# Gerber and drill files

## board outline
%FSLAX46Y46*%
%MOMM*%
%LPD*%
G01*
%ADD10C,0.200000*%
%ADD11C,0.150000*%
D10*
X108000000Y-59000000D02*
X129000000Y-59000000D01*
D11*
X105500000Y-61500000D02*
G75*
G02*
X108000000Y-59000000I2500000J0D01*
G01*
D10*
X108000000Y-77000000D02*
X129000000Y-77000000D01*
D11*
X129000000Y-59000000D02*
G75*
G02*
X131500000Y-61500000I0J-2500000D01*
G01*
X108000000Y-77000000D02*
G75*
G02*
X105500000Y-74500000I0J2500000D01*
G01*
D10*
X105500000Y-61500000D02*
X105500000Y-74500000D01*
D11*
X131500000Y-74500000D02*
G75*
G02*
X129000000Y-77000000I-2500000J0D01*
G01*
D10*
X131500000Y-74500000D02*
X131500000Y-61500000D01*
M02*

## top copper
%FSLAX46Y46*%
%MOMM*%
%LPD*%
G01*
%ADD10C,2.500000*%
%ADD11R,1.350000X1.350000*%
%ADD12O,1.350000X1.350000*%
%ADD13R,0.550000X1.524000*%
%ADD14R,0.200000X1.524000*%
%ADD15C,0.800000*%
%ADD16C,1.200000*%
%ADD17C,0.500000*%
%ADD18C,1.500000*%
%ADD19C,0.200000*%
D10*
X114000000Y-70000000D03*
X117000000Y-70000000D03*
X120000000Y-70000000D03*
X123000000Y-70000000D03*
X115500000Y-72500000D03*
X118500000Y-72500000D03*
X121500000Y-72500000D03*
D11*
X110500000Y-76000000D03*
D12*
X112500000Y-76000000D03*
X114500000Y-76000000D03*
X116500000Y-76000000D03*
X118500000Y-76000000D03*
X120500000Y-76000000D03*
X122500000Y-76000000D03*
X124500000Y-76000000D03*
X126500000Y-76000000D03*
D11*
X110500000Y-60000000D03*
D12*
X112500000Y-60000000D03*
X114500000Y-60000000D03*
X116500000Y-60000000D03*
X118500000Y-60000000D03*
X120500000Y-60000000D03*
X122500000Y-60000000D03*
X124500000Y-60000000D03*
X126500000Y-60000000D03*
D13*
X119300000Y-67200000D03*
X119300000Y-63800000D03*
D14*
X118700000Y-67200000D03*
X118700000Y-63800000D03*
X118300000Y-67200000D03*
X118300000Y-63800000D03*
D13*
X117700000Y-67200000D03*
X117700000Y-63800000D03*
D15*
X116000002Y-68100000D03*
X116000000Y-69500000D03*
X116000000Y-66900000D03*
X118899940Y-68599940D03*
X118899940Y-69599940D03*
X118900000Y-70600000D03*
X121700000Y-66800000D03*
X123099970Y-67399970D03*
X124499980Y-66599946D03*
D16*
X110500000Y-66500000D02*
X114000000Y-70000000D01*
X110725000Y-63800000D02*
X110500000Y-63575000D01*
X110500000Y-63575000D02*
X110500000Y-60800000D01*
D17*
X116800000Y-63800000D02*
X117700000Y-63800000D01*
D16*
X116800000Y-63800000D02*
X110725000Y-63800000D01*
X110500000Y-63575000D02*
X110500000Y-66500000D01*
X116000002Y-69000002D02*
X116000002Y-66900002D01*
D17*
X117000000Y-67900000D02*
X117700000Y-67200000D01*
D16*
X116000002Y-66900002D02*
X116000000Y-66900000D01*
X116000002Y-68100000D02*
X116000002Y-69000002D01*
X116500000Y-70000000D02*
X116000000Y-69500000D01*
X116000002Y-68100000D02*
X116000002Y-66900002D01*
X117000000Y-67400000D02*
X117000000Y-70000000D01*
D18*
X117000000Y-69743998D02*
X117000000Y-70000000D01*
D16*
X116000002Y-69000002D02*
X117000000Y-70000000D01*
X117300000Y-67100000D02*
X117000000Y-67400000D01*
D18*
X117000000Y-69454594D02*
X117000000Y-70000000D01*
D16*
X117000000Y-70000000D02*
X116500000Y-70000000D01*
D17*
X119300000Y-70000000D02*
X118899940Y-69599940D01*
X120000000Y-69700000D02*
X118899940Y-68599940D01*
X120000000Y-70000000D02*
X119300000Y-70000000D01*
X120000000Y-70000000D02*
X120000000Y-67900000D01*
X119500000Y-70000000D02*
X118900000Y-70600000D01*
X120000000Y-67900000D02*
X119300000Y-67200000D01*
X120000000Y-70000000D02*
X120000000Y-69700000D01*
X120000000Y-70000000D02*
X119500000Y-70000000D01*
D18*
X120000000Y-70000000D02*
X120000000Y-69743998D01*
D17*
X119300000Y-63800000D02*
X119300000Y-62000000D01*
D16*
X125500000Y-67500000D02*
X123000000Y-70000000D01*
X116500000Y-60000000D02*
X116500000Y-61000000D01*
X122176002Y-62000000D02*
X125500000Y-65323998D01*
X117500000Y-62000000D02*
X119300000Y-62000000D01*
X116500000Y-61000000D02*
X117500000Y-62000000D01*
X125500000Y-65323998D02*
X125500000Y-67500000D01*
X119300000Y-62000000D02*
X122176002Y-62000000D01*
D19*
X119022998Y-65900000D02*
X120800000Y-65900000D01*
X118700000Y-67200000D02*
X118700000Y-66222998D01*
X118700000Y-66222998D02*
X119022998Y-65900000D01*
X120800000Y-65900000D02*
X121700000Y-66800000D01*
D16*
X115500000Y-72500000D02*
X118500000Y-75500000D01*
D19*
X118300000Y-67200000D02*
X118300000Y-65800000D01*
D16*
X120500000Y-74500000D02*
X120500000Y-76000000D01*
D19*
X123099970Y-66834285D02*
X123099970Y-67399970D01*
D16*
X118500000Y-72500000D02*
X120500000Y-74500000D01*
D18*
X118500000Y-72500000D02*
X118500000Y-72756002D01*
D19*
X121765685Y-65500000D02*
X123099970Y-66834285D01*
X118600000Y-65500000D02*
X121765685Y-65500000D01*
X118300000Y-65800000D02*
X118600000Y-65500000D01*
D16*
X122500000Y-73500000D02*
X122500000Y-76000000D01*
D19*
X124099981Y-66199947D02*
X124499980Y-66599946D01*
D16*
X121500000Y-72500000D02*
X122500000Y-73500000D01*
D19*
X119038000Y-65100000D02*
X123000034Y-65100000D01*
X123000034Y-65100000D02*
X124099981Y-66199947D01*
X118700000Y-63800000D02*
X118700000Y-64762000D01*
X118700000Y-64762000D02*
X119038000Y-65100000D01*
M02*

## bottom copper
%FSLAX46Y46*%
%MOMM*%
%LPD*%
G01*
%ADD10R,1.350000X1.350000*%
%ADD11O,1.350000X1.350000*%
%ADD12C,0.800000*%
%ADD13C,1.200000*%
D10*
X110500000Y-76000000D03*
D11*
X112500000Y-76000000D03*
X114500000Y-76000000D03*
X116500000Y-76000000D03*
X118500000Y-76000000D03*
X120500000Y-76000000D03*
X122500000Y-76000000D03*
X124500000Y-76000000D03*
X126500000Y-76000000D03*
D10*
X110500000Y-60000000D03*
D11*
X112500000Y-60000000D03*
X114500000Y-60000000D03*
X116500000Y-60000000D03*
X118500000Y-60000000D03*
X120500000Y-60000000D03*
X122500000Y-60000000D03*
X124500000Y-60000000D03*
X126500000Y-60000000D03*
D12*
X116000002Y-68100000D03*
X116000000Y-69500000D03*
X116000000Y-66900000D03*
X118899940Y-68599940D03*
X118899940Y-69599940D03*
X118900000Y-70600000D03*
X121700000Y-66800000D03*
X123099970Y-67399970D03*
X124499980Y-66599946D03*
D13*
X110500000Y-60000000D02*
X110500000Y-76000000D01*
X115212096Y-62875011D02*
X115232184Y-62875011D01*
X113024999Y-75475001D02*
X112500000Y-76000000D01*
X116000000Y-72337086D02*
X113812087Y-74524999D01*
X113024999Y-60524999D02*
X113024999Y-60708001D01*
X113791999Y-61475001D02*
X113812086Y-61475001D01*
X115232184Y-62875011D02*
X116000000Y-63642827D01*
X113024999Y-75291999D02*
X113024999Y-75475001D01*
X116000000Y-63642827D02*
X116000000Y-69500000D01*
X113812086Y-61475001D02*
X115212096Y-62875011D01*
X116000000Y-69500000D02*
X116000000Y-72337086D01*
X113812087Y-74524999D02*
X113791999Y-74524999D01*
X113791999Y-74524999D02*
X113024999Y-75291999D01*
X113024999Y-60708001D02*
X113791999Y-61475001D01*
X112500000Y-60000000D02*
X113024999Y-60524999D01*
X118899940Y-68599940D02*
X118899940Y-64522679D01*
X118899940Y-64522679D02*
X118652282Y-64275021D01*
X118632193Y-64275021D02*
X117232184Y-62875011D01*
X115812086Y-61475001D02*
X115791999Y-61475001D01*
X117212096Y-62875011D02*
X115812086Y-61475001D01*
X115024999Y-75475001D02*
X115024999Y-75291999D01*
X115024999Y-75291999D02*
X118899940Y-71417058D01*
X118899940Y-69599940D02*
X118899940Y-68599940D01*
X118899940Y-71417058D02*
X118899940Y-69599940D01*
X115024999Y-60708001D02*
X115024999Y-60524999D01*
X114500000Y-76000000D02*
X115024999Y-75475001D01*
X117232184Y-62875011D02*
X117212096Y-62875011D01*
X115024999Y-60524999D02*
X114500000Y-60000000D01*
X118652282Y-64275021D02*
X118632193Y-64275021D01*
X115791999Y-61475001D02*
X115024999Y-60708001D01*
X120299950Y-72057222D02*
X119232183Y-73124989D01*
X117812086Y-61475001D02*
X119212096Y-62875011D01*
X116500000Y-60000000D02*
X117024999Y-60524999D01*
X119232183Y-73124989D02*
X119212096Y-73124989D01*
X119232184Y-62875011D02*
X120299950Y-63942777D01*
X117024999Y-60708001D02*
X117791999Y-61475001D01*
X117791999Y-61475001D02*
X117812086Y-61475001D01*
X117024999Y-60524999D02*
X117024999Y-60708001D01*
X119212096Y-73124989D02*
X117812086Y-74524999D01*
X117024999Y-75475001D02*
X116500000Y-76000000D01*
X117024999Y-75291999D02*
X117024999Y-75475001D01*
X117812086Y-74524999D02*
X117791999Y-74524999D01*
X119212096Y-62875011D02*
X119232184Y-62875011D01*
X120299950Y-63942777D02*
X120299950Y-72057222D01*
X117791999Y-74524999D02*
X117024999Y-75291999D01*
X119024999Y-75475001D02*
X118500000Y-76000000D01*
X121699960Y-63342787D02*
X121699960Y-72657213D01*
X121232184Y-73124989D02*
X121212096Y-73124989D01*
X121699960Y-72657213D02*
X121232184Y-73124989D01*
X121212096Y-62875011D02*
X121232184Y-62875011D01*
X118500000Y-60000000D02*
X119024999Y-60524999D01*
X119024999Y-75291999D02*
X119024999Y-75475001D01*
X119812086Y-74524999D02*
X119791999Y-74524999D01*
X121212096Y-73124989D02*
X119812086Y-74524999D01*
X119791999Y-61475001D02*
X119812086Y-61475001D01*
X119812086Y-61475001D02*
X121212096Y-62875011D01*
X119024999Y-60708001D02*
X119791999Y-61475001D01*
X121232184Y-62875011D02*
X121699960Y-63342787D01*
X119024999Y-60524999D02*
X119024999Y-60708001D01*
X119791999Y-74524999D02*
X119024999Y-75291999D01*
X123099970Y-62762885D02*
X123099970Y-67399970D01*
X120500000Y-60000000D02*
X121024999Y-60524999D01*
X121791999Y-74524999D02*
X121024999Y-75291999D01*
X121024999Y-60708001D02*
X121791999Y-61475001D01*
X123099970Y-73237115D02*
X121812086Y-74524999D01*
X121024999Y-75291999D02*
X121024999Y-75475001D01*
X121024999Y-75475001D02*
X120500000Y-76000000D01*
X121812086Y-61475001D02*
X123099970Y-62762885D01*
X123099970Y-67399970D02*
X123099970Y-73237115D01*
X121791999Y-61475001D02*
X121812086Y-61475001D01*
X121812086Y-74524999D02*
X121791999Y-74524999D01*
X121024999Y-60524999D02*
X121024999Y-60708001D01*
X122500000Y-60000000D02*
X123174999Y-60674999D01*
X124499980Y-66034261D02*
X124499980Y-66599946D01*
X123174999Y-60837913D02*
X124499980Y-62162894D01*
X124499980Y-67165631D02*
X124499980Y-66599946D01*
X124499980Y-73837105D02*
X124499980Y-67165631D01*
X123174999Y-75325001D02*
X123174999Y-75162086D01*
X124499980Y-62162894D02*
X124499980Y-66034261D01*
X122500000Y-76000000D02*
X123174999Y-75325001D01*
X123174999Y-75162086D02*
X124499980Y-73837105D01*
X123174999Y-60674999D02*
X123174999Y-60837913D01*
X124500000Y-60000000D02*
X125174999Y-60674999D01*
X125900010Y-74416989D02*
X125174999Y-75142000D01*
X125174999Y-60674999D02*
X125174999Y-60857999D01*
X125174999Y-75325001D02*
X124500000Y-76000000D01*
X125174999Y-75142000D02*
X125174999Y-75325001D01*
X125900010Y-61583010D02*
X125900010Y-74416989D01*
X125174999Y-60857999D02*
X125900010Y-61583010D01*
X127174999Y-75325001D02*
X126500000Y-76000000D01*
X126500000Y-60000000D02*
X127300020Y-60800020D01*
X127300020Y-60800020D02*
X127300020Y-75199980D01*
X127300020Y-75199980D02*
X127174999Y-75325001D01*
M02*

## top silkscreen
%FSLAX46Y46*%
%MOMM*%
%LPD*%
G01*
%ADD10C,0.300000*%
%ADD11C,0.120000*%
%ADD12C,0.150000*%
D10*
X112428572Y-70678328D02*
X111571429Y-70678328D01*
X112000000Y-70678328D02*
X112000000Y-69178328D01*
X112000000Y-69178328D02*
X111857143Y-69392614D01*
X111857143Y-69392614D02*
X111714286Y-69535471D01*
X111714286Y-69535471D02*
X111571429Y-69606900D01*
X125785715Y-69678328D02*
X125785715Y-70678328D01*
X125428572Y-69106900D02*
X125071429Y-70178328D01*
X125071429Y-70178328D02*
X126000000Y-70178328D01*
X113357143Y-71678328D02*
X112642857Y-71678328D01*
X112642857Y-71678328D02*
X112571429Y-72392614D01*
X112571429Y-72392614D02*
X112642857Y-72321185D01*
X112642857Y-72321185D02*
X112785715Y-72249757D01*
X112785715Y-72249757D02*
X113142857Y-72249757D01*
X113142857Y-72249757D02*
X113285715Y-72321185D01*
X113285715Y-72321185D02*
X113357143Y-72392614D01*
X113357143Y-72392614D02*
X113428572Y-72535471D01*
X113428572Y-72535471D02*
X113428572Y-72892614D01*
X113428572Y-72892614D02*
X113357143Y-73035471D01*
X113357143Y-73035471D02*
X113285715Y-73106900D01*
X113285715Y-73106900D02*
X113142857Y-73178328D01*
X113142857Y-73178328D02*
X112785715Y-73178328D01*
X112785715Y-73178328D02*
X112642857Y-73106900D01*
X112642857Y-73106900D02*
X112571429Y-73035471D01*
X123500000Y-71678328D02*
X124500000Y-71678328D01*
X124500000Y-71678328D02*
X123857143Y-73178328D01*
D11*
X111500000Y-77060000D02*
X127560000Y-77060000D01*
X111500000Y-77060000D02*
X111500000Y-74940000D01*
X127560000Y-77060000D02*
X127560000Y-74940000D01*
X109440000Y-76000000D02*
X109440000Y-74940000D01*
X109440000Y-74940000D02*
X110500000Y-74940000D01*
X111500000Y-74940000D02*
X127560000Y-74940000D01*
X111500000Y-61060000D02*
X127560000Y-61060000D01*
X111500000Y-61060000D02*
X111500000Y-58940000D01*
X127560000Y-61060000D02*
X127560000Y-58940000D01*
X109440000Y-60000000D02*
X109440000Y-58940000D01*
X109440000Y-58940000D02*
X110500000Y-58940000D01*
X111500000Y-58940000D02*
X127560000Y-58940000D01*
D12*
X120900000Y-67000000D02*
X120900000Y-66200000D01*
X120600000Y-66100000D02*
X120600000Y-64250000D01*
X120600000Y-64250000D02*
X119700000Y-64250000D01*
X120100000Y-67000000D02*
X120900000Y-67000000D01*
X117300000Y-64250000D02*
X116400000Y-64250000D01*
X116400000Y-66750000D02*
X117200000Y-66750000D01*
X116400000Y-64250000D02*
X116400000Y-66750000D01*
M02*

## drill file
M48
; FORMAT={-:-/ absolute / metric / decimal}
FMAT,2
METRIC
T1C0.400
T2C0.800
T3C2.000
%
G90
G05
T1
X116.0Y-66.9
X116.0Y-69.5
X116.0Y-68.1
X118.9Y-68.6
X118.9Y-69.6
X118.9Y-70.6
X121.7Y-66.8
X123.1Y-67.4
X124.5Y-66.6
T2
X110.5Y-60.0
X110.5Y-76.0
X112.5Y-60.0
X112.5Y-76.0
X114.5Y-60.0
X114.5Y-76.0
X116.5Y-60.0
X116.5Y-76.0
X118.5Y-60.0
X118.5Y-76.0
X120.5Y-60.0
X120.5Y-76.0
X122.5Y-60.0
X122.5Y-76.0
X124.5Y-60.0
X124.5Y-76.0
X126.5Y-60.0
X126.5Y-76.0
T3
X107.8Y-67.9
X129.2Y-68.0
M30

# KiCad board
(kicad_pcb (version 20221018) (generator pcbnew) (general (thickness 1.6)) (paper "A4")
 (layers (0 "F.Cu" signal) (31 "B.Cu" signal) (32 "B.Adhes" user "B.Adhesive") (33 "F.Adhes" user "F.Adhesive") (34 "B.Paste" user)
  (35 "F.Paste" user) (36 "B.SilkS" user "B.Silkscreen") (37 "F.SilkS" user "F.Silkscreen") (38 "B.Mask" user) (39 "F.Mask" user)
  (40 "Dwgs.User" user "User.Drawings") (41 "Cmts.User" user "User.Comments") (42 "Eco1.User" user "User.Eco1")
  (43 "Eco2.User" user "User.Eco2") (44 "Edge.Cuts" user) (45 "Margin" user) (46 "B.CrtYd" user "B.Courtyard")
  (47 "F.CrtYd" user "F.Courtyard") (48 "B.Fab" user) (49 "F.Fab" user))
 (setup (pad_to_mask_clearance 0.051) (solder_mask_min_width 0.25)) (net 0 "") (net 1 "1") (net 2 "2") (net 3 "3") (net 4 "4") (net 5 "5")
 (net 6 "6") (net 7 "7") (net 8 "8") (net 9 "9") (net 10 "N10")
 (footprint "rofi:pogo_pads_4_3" (layer "F.Cu") (at 118.5 70)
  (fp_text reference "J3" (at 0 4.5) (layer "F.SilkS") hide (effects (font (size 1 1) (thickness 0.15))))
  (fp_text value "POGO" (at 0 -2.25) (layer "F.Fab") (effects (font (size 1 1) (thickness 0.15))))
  (pad "1" smd circle (at -4.5 0) (size 2.5 2.5) (layers "F.Cu" "F.Paste" "F.Mask") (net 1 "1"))
  (pad "2" smd circle (at -1.5 0) (size 2.5 2.5) (layers "F.Cu" "F.Paste" "F.Mask") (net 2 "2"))
  (pad "3" smd circle (at 1.5 0) (size 2.5 2.5) (layers "F.Cu" "F.Paste" "F.Mask") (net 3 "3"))
  (pad "4" smd circle (at 4.5 0) (size 2.5 2.5) (layers "F.Cu" "F.Paste" "F.Mask") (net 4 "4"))
  (pad "5" smd circle (at -3 2.5) (size 2.5 2.5) (layers "F.Cu" "F.Paste" "F.Mask") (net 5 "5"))
  (pad "6" smd circle (at 0 2.5) (size 2.5 2.5) (layers "F.Cu" "F.Paste" "F.Mask") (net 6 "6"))
  (pad "7" smd circle (at 3 2.5) (size 2.5 2.5) (layers "F.Cu" "F.Paste" "F.Mask") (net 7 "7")))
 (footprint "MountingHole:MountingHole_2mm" (layer "F.Cu") (at 129.2 68)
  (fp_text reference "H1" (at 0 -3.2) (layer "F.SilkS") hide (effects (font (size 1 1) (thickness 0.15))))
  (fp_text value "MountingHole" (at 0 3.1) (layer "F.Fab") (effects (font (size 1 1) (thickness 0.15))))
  (pad "" np_thru_hole circle (at 0 0) (size 2 2) (drill 2) (layers "*.Cu" "*.Mask")))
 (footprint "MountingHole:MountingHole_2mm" (layer "F.Cu") (at 107.8 67.9)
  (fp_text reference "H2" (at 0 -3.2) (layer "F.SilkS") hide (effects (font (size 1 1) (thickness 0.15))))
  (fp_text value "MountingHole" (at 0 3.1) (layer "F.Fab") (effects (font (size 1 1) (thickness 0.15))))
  (pad "" np_thru_hole circle (at 0 0) (size 2 2) (drill 2) (layers "*.Cu" "*.Mask")))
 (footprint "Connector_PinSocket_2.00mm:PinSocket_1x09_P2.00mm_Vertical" (layer "F.Cu") (at 110.5 76 90)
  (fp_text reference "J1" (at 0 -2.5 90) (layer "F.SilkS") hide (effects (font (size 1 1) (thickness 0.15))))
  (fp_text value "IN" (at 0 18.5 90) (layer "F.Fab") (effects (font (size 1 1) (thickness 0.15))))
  (fp_line (start -1.06 1) (end -1.06 17.06) (stroke (width 0.12) (type solid)) (layer "F.SilkS"))
  (fp_line (start -1.06 1) (end 1.06 1) (stroke (width 0.12) (type solid)) (layer "F.SilkS"))
  (fp_line (start -1.06 17.06) (end 1.06 17.06) (stroke (width 0.12) (type solid)) (layer "F.SilkS"))
  (fp_line (start 0 -1.06) (end 1.06 -1.06) (stroke (width 0.12) (type solid)) (layer "F.SilkS"))
  (fp_line (start 1.06 -1.06) (end 1.06 0) (stroke (width 0.12) (type solid)) (layer "F.SilkS"))
  (fp_line (start 1.06 1) (end 1.06 17.06) (stroke (width 0.12) (type solid)) (layer "F.SilkS"))
  (pad "1" thru_hole rect (at 0 0 90) (size 1.35 1.35) (drill 0.8) (layers "*.Cu" "*.Mask") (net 1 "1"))
  (pad "2" thru_hole oval (at 0 2 90) (size 1.35 1.35) (drill 0.8) (layers "*.Cu" "*.Mask") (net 2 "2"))
  (pad "3" thru_hole oval (at 0 4 90) (size 1.35 1.35) (drill 0.8) (layers "*.Cu" "*.Mask") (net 3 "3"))
  (pad "4" thru_hole oval (at 0 6 90) (size 1.35 1.35) (drill 0.8) (layers "*.Cu" "*.Mask") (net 4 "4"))
  (pad "5" thru_hole oval (at 0 8 90) (size 1.35 1.35) (drill 0.8) (layers "*.Cu" "*.Mask") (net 5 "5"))
  (pad "6" thru_hole oval (at 0 10 90) (size 1.35 1.35) (drill 0.8) (layers "*.Cu" "*.Mask") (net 6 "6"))
  (pad "7" thru_hole oval (at 0 12 90) (size 1.35 1.35) (drill 0.8) (layers "*.Cu" "*.Mask") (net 7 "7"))
  (pad "8" thru_hole oval (at 0 14 90) (size 1.35 1.35) (drill 0.8) (layers "*.Cu" "*.Mask") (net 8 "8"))
  (pad "9" thru_hole oval (at 0 16 90) (size 1.35 1.35) (drill 0.8) (layers "*.Cu" "*.Mask") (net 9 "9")))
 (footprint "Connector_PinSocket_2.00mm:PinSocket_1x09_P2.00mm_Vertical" (layer "F.Cu") (at 110.5 60 90)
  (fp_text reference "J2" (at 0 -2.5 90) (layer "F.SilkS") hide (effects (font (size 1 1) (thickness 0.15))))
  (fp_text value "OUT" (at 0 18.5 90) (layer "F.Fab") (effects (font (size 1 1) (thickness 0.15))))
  (fp_line (start -1.06 1) (end -1.06 17.06) (stroke (width 0.12) (type solid)) (layer "F.SilkS"))
  (fp_line (start -1.06 1) (end 1.06 1) (stroke (width 0.12) (type solid)) (layer "F.SilkS"))
  (fp_line (start -1.06 17.06) (end 1.06 17.06) (stroke (width 0.12) (type solid)) (layer "F.SilkS"))
  (fp_line (start 0 -1.06) (end 1.06 -1.06) (stroke (width 0.12) (type solid)) (layer "F.SilkS"))
  (fp_line (start 1.06 -1.06) (end 1.06 0) (stroke (width 0.12) (type solid)) (layer "F.SilkS"))
  (fp_line (start 1.06 1) (end 1.06 17.06) (stroke (width 0.12) (type solid)) (layer "F.SilkS"))
  (pad "1" thru_hole rect (at 0 0 90) (size 1.35 1.35) (drill 0.8) (layers "*.Cu" "*.Mask") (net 1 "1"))
  (pad "2" thru_hole oval (at 0 2 90) (size 1.35 1.35) (drill 0.8) (layers "*.Cu" "*.Mask") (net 2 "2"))
  (pad "3" thru_hole oval (at 0 4 90) (size 1.35 1.35) (drill 0.8) (layers "*.Cu" "*.Mask") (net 3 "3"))
  (pad "4" thru_hole oval (at 0 6 90) (size 1.35 1.35) (drill 0.8) (layers "*.Cu" "*.Mask") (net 4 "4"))
  (pad "5" thru_hole oval (at 0 8 90) (size 1.35 1.35) (drill 0.8) (layers "*.Cu" "*.Mask") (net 5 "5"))
  (pad "6" thru_hole oval (at 0 10 90) (size 1.35 1.35) (drill 0.8) (layers "*.Cu" "*.Mask") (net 6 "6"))
  (pad "7" thru_hole oval (at 0 12 90) (size 1.35 1.35) (drill 0.8) (layers "*.Cu" "*.Mask") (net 7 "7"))
  (pad "8" thru_hole oval (at 0 14 90) (size 1.35 1.35) (drill 0.8) (layers "*.Cu" "*.Mask") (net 8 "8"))
  (pad "9" thru_hole oval (at 0 16 90) (size 1.35 1.35) (drill 0.8) (layers "*.Cu" "*.Mask") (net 9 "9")))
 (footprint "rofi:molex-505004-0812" (layer "F.Cu") (at 118.5 65.5 180)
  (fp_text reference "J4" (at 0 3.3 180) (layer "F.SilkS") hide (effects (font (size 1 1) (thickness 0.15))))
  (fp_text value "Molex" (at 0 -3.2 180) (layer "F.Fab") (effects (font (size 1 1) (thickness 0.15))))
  (fp_line (start -2.4 -1.5) (end -2.4 -0.7) (stroke (width 0.15) (type solid)) (layer "F.SilkS"))
  (fp_line (start -2.1 -0.6) (end -2.1 1.25) (stroke (width 0.15) (type solid)) (layer "F.SilkS"))
  (fp_line (start -2.1 1.25) (end -1.2 1.25) (stroke (width 0.15) (type solid)) (layer "F.SilkS"))
  (fp_line (start -1.6 -1.5) (end -2.4 -1.5) (stroke (width 0.15) (type solid)) (layer "F.SilkS"))
  (fp_line (start 1.2 1.25) (end 2.1 1.25) (stroke (width 0.15) (type solid)) (layer "F.SilkS"))
  (fp_line (start 2.1 -1.25) (end 1.3 -1.25) (stroke (width 0.15) (type solid)) (layer "F.SilkS"))
  (fp_line (start 2.1 1.25) (end 2.1 -1.25) (stroke (width 0.15) (type solid)) (layer "F.SilkS"))
  (pad "1" smd rect (at -0.8 -1.7 180) (size 0.55 1.524) (layers "F.Cu" "F.Paste" "F.Mask") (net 3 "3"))
  (pad "2" smd rect (at -0.8 1.7 180) (size 0.55 1.524) (layers "F.Cu" "F.Paste" "F.Mask") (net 4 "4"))
  (pad "3" smd rect (at -0.2 -1.7 180) (size 0.2 1.524) (layers "F.Cu" "F.Paste" "F.Mask") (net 5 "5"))
  (pad "4" smd rect (at -0.2 1.7 180) (size 0.2 1.524) (layers "F.Cu" "F.Paste" "F.Mask") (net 7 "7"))
  (pad "5" smd rect (at 0.2 -1.7 180) (size 0.2 1.524) (layers "F.Cu" "F.Paste" "F.Mask") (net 6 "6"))
  (pad "6" smd rect (at 0.2 1.7 180) (size 0.2 1.524) (layers "F.Cu" "F.Paste" "F.Mask") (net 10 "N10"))
  (pad "7" smd rect (at 0.8 -1.7 180) (size 0.55 1.524) (layers "F.Cu" "F.Paste" "F.Mask") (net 2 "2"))
  (pad "8" smd rect (at 0.8 1.7 180) (size 0.55 1.524) (layers "F.Cu" "F.Paste" "F.Mask") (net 1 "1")))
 (gr_line (start 108 59) (end 129 59) (stroke (width 0.2) (type solid)) (layer "Edge.Cuts"))
 (gr_arc (start 105.5 61.5) (mid 106.232233 59.732233) (end 108 59) (stroke (width 0.15) (type solid)) (layer "Edge.Cuts"))
 (gr_line (start 108 77) (end 129 77) (stroke (width 0.2) (type solid)) (layer "Edge.Cuts"))
 (gr_arc (start 129 59) (mid 130.767767 59.732233) (end 131.5 61.5) (stroke (width 0.15) (type solid)) (layer "Edge.Cuts"))
 (gr_arc (start 108 77) (mid 106.232233 76.267767) (end 105.5 74.5) (stroke (width 0.15) (type solid)) (layer "Edge.Cuts"))
 (gr_line (start 105.5 61.5) (end 105.5 74.5) (stroke (width 0.2) (type solid)) (layer "Edge.Cuts"))
 (gr_arc (start 131.5 74.5) (mid 130.767767 76.267767) (end 129 77) (stroke (width 0.15) (type solid)) (layer "Edge.Cuts"))
 (gr_line (start 131.5 74.5) (end 131.5 61.5) (stroke (width 0.2) (type solid)) (layer "Edge.Cuts"))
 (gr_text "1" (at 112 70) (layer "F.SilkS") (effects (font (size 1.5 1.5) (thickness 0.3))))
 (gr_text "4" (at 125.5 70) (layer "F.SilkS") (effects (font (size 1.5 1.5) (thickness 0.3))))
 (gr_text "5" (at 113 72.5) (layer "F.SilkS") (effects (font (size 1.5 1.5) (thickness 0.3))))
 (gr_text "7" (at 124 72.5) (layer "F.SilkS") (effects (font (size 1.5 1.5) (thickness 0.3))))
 (segment (start 110.5 66.5) (end 114 70) (width 1.2) (layer "F.Cu") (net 1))
 (segment (start 110.725 63.8) (end 110.5 63.575) (width 1.2) (layer "F.Cu") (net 1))
 (segment (start 110.5 63.575) (end 110.5 60.8) (width 1.2) (layer "F.Cu") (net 1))
 (segment (start 116.8 63.8) (end 117.7 63.8) (width 0.5) (layer "F.Cu") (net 1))
 (segment (start 116.8 63.8) (end 110.725 63.8) (width 1.2) (layer "F.Cu") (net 1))
 (segment (start 110.5 63.575) (end 110.5 66.5) (width 1.2) (layer "F.Cu") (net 1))
 (segment (start 110.5 60) (end 110.5 76) (width 1.2) (layer "B.Cu") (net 1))
 (segment (start 116.000002 69.000002) (end 116.000002 66.900002) (width 1.2) (layer "F.Cu") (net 2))
 (segment (start 117 67.9) (end 117.7 67.2) (width 0.5) (layer "F.Cu") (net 2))
 (segment (start 116.000002 66.900002) (end 116 66.9) (width 1.2) (layer "F.Cu") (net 2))
 (segment (start 116.000002 68.1) (end 116.000002 69.000002) (width 1.2) (layer "F.Cu") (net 2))
 (segment (start 116.5 70) (end 116 69.5) (width 1.2) (layer "F.Cu") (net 2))
 (segment (start 116.000002 68.1) (end 116.000002 66.900002) (width 1.2) (layer "F.Cu") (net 2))
 (segment (start 117 67.4) (end 117 70) (width 1.2) (layer "F.Cu") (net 2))
 (segment (start 117 69.743998) (end 117 70) (width 1.5) (layer "F.Cu") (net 2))
 (segment (start 116.000002 69.000002) (end 117 70) (width 1.2) (layer "F.Cu") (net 2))
 (segment (start 117.3 67.1) (end 117 67.4) (width 1.2) (layer "F.Cu") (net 2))
 (segment (start 117 69.454594) (end 117 70) (width 1.5) (layer "F.Cu") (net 2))
 (segment (start 117 70) (end 116.5 70) (width 1.2) (layer "F.Cu") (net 2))
 (via (at 116.000002 68.1) (size 0.8) (drill 0.4) (layers "F.Cu" "B.Cu") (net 2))
 (via (at 116 69.5) (size 0.8) (drill 0.4) (layers "F.Cu" "B.Cu") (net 2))
 (via (at 116 66.9) (size 0.8) (drill 0.4) (layers "F.Cu" "B.Cu") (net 2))
 (segment (start 115.212096 62.875011) (end 115.232184 62.875011) (width 1.2) (layer "B.Cu") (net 2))
 (segment (start 113.024999 75.475001) (end 112.5 76) (width 1.2) (layer "B.Cu") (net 2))
 (segment (start 116 72.337086) (end 113.812087 74.524999) (width 1.2) (layer "B.Cu") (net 2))
 (segment (start 113.024999 60.524999) (end 113.024999 60.708001) (width 1.2) (layer "B.Cu") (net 2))
 (segment (start 113.791999 61.475001) (end 113.812086 61.475001) (width 1.2) (layer "B.Cu") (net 2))
 (segment (start 115.232184 62.875011) (end 116 63.642827) (width 1.2) (layer "B.Cu") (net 2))
 (segment (start 113.024999 75.291999) (end 113.024999 75.475001) (width 1.2) (layer "B.Cu") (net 2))
 (segment (start 116 63.642827) (end 116 69.5) (width 1.2) (layer "B.Cu") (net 2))
 (segment (start 113.812086 61.475001) (end 115.212096 62.875011) (width 1.2) (layer "B.Cu") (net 2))
 (segment (start 116 69.5) (end 116 72.337086) (width 1.2) (layer "B.Cu") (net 2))
 (segment (start 113.812087 74.524999) (end 113.791999 74.524999) (width 1.2) (layer "B.Cu") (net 2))
 (segment (start 113.791999 74.524999) (end 113.024999 75.291999) (width 1.2) (layer "B.Cu") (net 2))
 (segment (start 113.024999 60.708001) (end 113.791999 61.475001) (width 1.2) (layer "B.Cu") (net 2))
 (segment (start 112.5 60) (end 113.024999 60.524999) (width 1.2) (layer "B.Cu") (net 2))
 (segment (start 119.3 70) (end 118.89994 69.59994) (width 0.5) (layer "F.Cu") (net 3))
 (segment (start 120 69.7) (end 118.89994 68.59994) (width 0.5) (layer "F.Cu") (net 3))
 (segment (start 120 70) (end 119.3 70) (width 0.5) (layer "F.Cu") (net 3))
 (segment (start 120 70) (end 120 67.9) (width 0.5) (layer "F.Cu") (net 3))
 (segment (start 119.5 70) (end 118.9 70.6) (width 0.5) (layer "F.Cu") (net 3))
 (segment (start 120 67.9) (end 119.3 67.2) (width 0.5) (layer "F.Cu") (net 3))
 (segment (start 120 70) (end 120 69.7) (width 0.5) (layer "F.Cu") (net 3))
 (segment (start 120 70) (end 119.5 70) (width 0.5) (layer "F.Cu") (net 3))
 (segment (start 120 70) (end 120 69.743998) (width 1.5) (layer "F.Cu") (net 3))
 (via (at 118.89994 68.59994) (size 0.8) (drill 0.4) (layers "F.Cu" "B.Cu") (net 3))
 (via (at 118.89994 69.59994) (size 0.8) (drill 0.4) (layers "F.Cu" "B.Cu") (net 3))
 (via (at 118.9 70.6) (size 0.8) (drill 0.4) (layers "F.Cu" "B.Cu") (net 3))
 (segment (start 118.89994 68.59994) (end 118.89994 64.522679) (width 1.2) (layer "B.Cu") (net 3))
 (segment (start 118.89994 64.522679) (end 118.652282 64.275021) (width 1.2) (layer "B.Cu") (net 3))
 (segment (start 118.632193 64.275021) (end 117.232184 62.875011) (width 1.2) (layer "B.Cu") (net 3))
 (segment (start 115.812086 61.475001) (end 115.791999 61.475001) (width 1.2) (layer "B.Cu") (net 3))
 (segment (start 117.212096 62.875011) (end 115.812086 61.475001) (width 1.2) (layer "B.Cu") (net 3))
 (segment (start 115.024999 75.475001) (end 115.024999 75.291999) (width 1.2) (layer "B.Cu") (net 3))
 (segment (start 115.024999 75.291999) (end 118.89994 71.417058) (width 1.2) (layer "B.Cu") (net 3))
 (segment (start 118.89994 69.59994) (end 118.89994 68.59994) (width 1.2) (layer "B.Cu") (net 3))
 (segment (start 118.89994 71.417058) (end 118.89994 69.59994) (width 1.2) (layer "B.Cu") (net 3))
 (segment (start 115.024999 60.708001) (end 115.024999 60.524999) (width 1.2) (layer "B.Cu") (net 3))
 (segment (start 114.5 76) (end 115.024999 75.475001) (width 1.2) (layer "B.Cu") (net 3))
 (segment (start 117.232184 62.875011) (end 117.212096 62.875011) (width 1.2) (layer "B.Cu") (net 3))
 (segment (start 115.024999 60.524999) (end 114.5 60) (width 1.2) (layer "B.Cu") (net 3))
 (segment (start 118.652282 64.275021) (end 118.632193 64.275021) (width 1.2) (layer "B.Cu") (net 3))
 (segment (start 115.791999 61.475001) (end 115.024999 60.708001) (width 1.2) (layer "B.Cu") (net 3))
 (segment (start 119.3 63.8) (end 119.3 62) (width 0.5) (layer "F.Cu") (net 4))
 (segment (start 125.5 67.5) (end 123 70) (width 1.2) (layer "F.Cu") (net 4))
 (segment (start 116.5 60) (end 116.5 61) (width 1.2) (layer "F.Cu") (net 4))
 (segment (start 122.176002 62) (end 125.5 65.323998) (width 1.2) (layer "F.Cu") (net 4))
 (segment (start 117.5 62) (end 119.3 62) (width 1.2) (layer "F.Cu") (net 4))
 (segment (start 116.5 61) (end 117.5 62) (width 1.2) (layer "F.Cu") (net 4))
 (segment (start 125.5 65.323998) (end 125.5 67.5) (width 1.2) (layer "F.Cu") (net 4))
 (segment (start 119.3 62) (end 122.176002 62) (width 1.2) (layer "F.Cu") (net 4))
 (segment (start 120.29995 72.057222) (end 119.232183 73.124989) (width 1.2) (layer "B.Cu") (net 4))
 (segment (start 117.812086 61.475001) (end 119.212096 62.875011) (width 1.2) (layer "B.Cu") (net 4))
 (segment (start 116.5 60) (end 117.024999 60.524999) (width 1.2) (layer "B.Cu") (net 4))
 (segment (start 119.232183 73.124989) (end 119.212096 73.124989) (width 1.2) (layer "B.Cu") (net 4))
 (segment (start 119.232184 62.875011) (end 120.29995 63.942777) (width 1.2) (layer "B.Cu") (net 4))
 (segment (start 117.024999 60.708001) (end 117.791999 61.475001) (width 1.2) (layer "B.Cu") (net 4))
 (segment (start 117.791999 61.475001) (end 117.812086 61.475001) (width 1.2) (layer "B.Cu") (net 4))
 (segment (start 117.024999 60.524999) (end 117.024999 60.708001) (width 1.2) (layer "B.Cu") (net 4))
 (segment (start 119.212096 73.124989) (end 117.812086 74.524999) (width 1.2) (layer "B.Cu") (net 4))
 (segment (start 117.024999 75.475001) (end 116.5 76) (width 1.2) (layer "B.Cu") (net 4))
 (segment (start 117.024999 75.291999) (end 117.024999 75.475001) (width 1.2) (layer "B.Cu") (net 4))
 (segment (start 117.812086 74.524999) (end 117.791999 74.524999) (width 1.2) (layer "B.Cu") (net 4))
 (segment (start 119.212096 62.875011) (end 119.232184 62.875011) (width 1.2) (layer "B.Cu") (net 4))
 (segment (start 120.29995 63.942777) (end 120.29995 72.057222) (width 1.2) (layer "B.Cu") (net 4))
 (segment (start 117.791999 74.524999) (end 117.024999 75.291999) (width 1.2) (layer "B.Cu") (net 4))
 (segment (start 119.022998 65.9) (end 120.8 65.9) (width 0.2) (layer "F.Cu") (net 5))
 (segment (start 118.7 67.2) (end 118.7 66.222998) (width 0.2) (layer "F.Cu") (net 5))
 (segment (start 118.7 66.222998) (end 119.022998 65.9) (width 0.2) (layer "F.Cu") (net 5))
 (segment (start 120.8 65.9) (end 121.7 66.8) (width 0.2) (layer "F.Cu") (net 5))
 (segment (start 115.5 72.5) (end 118.5 75.5) (width 1.2) (layer "F.Cu") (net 5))
 (via (at 121.7 66.8) (size 0.8) (drill 0.4) (layers "F.Cu" "B.Cu") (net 5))
 (segment (start 119.024999 75.475001) (end 118.5 76) (width 1.2) (layer "B.Cu") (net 5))
 (segment (start 121.69996 63.342787) (end 121.69996 72.657213) (width 1.2) (layer "B.Cu") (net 5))
 (segment (start 121.232184 73.124989) (end 121.212096 73.124989) (width 1.2) (layer "B.Cu") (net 5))
 (segment (start 121.69996 72.657213) (end 121.232184 73.124989) (width 1.2) (layer "B.Cu") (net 5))
 (segment (start 121.212096 62.875011) (end 121.232184 62.875011) (width 1.2) (layer "B.Cu") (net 5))
 (segment (start 118.5 60) (end 119.024999 60.524999) (width 1.2) (layer "B.Cu") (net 5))
 (segment (start 119.024999 75.291999) (end 119.024999 75.475001) (width 1.2) (layer "B.Cu") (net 5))
 (segment (start 119.812086 74.524999) (end 119.791999 74.524999) (width 1.2) (layer "B.Cu") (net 5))
 (segment (start 121.212096 73.124989) (end 119.812086 74.524999) (width 1.2) (layer "B.Cu") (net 5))
 (segment (start 119.791999 61.475001) (end 119.812086 61.475001) (width 1.2) (layer "B.Cu") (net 5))
 (segment (start 119.812086 61.475001) (end 121.212096 62.875011) (width 1.2) (layer "B.Cu") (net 5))
 (segment (start 119.024999 60.708001) (end 119.791999 61.475001) (width 1.2) (layer "B.Cu") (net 5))
 (segment (start 121.232184 62.875011) (end 121.69996 63.342787) (width 1.2) (layer "B.Cu") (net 5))
 (segment (start 119.024999 60.524999) (end 119.024999 60.708001) (width 1.2) (layer "B.Cu") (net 5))
 (segment (start 119.791999 74.524999) (end 119.024999 75.291999) (width 1.2) (layer "B.Cu") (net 5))
 (segment (start 118.3 67.2) (end 118.3 65.8) (width 0.2) (layer "F.Cu") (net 6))
 (segment (start 120.5 74.5) (end 120.5 76) (width 1.2) (layer "F.Cu") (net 6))
 (segment (start 123.09997 66.834285) (end 123.09997 67.39997) (width 0.2) (layer "F.Cu") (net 6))
 (segment (start 118.5 72.5) (end 120.5 74.5) (width 1.2) (layer "F.Cu") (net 6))
 (segment (start 118.5 72.5) (end 118.5 72.756002) (width 1.5) (layer "F.Cu") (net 6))
 (segment (start 121.765685 65.5) (end 123.09997 66.834285) (width 0.2) (layer "F.Cu") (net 6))
 (segment (start 118.6 65.5) (end 121.765685 65.5) (width 0.2) (layer "F.Cu") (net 6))
 (segment (start 118.3 65.8) (end 118.6 65.5) (width 0.2) (layer "F.Cu") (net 6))
 (via (at 123.09997 67.39997) (size 0.8) (drill 0.4) (layers "F.Cu" "B.Cu") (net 6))
 (segment (start 123.09997 62.762885) (end 123.09997 67.39997) (width 1.2) (layer "B.Cu") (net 6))
 (segment (start 120.5 60) (end 121.024999 60.524999) (width 1.2) (layer "B.Cu") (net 6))
 (segment (start 121.791999 74.524999) (end 121.024999 75.291999) (width 1.2) (layer "B.Cu") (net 6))
 (segment (start 121.024999 60.708001) (end 121.791999 61.475001) (width 1.2) (layer "B.Cu") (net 6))
 (segment (start 123.09997 73.237115) (end 121.812086 74.524999) (width 1.2) (layer "B.Cu") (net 6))
 (segment (start 121.024999 75.291999) (end 121.024999 75.475001) (width 1.2) (layer "B.Cu") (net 6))
 (segment (start 121.024999 75.475001) (end 120.5 76) (width 1.2) (layer "B.Cu") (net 6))
 (segment (start 121.812086 61.475001) (end 123.09997 62.762885) (width 1.2) (layer "B.Cu") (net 6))
 (segment (start 123.09997 67.39997) (end 123.09997 73.237115) (width 1.2) (layer "B.Cu") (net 6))
 (segment (start 121.791999 61.475001) (end 121.812086 61.475001) (width 1.2) (layer "B.Cu") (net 6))
 (segment (start 121.812086 74.524999) (end 121.791999 74.524999) (width 1.2) (layer "B.Cu") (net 6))
 (segment (start 121.024999 60.524999) (end 121.024999 60.708001) (width 1.2) (layer "B.Cu") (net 6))
 (segment (start 122.5 73.5) (end 122.5 76) (width 1.2) (layer "F.Cu") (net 7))
 (segment (start 124.099981 66.199947) (end 124.49998 66.599946) (width 0.2) (layer "F.Cu") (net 7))
 (segment (start 121.5 72.5) (end 122.5 73.5) (width 1.2) (layer "F.Cu") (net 7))
 (segment (start 119.038 65.1) (end 123.000034 65.1) (width 0.2) (layer "F.Cu") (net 7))
 (segment (start 123.000034 65.1) (end 124.099981 66.199947) (width 0.2) (layer "F.Cu") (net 7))
 (segment (start 118.7 63.8) (end 118.7 64.762) (width 0.2) (layer "F.Cu") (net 7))
 (segment (start 118.7 64.762) (end 119.038 65.1) (width 0.2) (layer "F.Cu") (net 7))
 (via (at 124.49998 66.599946) (size 0.8) (drill 0.4) (layers "F.Cu" "B.Cu") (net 7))
 (segment (start 122.5 60) (end 123.174999 60.674999) (width 1.2) (layer "B.Cu") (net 7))
 (segment (start 124.49998 66.034261) (end 124.49998 66.599946) (width 1.2) (layer "B.Cu") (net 7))
 (segment (start 123.174999 60.837913) (end 124.49998 62.162894) (width 1.2) (layer "B.Cu") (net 7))
 (segment (start 124.49998 67.165631) (end 124.49998 66.599946) (width 1.2) (layer "B.Cu") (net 7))
 (segment (start 124.49998 73.837105) (end 124.49998 67.165631) (width 1.2) (layer "B.Cu") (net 7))
 (segment (start 123.174999 75.325001) (end 123.174999 75.162086) (width 1.2) (layer "B.Cu") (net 7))
 (segment (start 124.49998 62.162894) (end 124.49998 66.034261) (width 1.2) (layer "B.Cu") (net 7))
 (segment (start 122.5 76) (end 123.174999 75.325001) (width 1.2) (layer "B.Cu") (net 7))
 (segment (start 123.174999 75.162086) (end 124.49998 73.837105) (width 1.2) (layer "B.Cu") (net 7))
 (segment (start 123.174999 60.674999) (end 123.174999 60.837913) (width 1.2) (layer "B.Cu") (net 7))
 (segment (start 124.5 60) (end 125.174999 60.674999) (width 1.2) (layer "B.Cu") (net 8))
 (segment (start 125.90001 74.416989) (end 125.174999 75.142) (width 1.2) (layer "B.Cu") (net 8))
 (segment (start 125.174999 60.674999) (end 125.174999 60.857999) (width 1.2) (layer "B.Cu") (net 8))
 (segment (start 125.174999 75.325001) (end 124.5 76) (width 1.2) (layer "B.Cu") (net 8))
 (segment (start 125.174999 75.142) (end 125.174999 75.325001) (width 1.2) (layer "B.Cu") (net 8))
 (segment (start 125.90001 61.58301) (end 125.90001 74.416989) (width 1.2) (layer "B.Cu") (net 8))
 (segment (start 125.174999 60.857999) (end 125.90001 61.58301) (width 1.2) (layer "B.Cu") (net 8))
 (segment (start 127.174999 75.325001) (end 126.5 76) (width 1.2) (layer "B.Cu") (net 9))
 (segment (start 126.5 60) (end 127.30002 60.80002) (width 1.2) (layer "B.Cu") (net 9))
 (segment (start 127.30002 60.80002) (end 127.30002 75.19998) (width 1.2) (layer "B.Cu") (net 9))
 (segment (start 127.30002 75.19998) (end 127.174999 75.325001) (width 1.2) (layer "B.Cu") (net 9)))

